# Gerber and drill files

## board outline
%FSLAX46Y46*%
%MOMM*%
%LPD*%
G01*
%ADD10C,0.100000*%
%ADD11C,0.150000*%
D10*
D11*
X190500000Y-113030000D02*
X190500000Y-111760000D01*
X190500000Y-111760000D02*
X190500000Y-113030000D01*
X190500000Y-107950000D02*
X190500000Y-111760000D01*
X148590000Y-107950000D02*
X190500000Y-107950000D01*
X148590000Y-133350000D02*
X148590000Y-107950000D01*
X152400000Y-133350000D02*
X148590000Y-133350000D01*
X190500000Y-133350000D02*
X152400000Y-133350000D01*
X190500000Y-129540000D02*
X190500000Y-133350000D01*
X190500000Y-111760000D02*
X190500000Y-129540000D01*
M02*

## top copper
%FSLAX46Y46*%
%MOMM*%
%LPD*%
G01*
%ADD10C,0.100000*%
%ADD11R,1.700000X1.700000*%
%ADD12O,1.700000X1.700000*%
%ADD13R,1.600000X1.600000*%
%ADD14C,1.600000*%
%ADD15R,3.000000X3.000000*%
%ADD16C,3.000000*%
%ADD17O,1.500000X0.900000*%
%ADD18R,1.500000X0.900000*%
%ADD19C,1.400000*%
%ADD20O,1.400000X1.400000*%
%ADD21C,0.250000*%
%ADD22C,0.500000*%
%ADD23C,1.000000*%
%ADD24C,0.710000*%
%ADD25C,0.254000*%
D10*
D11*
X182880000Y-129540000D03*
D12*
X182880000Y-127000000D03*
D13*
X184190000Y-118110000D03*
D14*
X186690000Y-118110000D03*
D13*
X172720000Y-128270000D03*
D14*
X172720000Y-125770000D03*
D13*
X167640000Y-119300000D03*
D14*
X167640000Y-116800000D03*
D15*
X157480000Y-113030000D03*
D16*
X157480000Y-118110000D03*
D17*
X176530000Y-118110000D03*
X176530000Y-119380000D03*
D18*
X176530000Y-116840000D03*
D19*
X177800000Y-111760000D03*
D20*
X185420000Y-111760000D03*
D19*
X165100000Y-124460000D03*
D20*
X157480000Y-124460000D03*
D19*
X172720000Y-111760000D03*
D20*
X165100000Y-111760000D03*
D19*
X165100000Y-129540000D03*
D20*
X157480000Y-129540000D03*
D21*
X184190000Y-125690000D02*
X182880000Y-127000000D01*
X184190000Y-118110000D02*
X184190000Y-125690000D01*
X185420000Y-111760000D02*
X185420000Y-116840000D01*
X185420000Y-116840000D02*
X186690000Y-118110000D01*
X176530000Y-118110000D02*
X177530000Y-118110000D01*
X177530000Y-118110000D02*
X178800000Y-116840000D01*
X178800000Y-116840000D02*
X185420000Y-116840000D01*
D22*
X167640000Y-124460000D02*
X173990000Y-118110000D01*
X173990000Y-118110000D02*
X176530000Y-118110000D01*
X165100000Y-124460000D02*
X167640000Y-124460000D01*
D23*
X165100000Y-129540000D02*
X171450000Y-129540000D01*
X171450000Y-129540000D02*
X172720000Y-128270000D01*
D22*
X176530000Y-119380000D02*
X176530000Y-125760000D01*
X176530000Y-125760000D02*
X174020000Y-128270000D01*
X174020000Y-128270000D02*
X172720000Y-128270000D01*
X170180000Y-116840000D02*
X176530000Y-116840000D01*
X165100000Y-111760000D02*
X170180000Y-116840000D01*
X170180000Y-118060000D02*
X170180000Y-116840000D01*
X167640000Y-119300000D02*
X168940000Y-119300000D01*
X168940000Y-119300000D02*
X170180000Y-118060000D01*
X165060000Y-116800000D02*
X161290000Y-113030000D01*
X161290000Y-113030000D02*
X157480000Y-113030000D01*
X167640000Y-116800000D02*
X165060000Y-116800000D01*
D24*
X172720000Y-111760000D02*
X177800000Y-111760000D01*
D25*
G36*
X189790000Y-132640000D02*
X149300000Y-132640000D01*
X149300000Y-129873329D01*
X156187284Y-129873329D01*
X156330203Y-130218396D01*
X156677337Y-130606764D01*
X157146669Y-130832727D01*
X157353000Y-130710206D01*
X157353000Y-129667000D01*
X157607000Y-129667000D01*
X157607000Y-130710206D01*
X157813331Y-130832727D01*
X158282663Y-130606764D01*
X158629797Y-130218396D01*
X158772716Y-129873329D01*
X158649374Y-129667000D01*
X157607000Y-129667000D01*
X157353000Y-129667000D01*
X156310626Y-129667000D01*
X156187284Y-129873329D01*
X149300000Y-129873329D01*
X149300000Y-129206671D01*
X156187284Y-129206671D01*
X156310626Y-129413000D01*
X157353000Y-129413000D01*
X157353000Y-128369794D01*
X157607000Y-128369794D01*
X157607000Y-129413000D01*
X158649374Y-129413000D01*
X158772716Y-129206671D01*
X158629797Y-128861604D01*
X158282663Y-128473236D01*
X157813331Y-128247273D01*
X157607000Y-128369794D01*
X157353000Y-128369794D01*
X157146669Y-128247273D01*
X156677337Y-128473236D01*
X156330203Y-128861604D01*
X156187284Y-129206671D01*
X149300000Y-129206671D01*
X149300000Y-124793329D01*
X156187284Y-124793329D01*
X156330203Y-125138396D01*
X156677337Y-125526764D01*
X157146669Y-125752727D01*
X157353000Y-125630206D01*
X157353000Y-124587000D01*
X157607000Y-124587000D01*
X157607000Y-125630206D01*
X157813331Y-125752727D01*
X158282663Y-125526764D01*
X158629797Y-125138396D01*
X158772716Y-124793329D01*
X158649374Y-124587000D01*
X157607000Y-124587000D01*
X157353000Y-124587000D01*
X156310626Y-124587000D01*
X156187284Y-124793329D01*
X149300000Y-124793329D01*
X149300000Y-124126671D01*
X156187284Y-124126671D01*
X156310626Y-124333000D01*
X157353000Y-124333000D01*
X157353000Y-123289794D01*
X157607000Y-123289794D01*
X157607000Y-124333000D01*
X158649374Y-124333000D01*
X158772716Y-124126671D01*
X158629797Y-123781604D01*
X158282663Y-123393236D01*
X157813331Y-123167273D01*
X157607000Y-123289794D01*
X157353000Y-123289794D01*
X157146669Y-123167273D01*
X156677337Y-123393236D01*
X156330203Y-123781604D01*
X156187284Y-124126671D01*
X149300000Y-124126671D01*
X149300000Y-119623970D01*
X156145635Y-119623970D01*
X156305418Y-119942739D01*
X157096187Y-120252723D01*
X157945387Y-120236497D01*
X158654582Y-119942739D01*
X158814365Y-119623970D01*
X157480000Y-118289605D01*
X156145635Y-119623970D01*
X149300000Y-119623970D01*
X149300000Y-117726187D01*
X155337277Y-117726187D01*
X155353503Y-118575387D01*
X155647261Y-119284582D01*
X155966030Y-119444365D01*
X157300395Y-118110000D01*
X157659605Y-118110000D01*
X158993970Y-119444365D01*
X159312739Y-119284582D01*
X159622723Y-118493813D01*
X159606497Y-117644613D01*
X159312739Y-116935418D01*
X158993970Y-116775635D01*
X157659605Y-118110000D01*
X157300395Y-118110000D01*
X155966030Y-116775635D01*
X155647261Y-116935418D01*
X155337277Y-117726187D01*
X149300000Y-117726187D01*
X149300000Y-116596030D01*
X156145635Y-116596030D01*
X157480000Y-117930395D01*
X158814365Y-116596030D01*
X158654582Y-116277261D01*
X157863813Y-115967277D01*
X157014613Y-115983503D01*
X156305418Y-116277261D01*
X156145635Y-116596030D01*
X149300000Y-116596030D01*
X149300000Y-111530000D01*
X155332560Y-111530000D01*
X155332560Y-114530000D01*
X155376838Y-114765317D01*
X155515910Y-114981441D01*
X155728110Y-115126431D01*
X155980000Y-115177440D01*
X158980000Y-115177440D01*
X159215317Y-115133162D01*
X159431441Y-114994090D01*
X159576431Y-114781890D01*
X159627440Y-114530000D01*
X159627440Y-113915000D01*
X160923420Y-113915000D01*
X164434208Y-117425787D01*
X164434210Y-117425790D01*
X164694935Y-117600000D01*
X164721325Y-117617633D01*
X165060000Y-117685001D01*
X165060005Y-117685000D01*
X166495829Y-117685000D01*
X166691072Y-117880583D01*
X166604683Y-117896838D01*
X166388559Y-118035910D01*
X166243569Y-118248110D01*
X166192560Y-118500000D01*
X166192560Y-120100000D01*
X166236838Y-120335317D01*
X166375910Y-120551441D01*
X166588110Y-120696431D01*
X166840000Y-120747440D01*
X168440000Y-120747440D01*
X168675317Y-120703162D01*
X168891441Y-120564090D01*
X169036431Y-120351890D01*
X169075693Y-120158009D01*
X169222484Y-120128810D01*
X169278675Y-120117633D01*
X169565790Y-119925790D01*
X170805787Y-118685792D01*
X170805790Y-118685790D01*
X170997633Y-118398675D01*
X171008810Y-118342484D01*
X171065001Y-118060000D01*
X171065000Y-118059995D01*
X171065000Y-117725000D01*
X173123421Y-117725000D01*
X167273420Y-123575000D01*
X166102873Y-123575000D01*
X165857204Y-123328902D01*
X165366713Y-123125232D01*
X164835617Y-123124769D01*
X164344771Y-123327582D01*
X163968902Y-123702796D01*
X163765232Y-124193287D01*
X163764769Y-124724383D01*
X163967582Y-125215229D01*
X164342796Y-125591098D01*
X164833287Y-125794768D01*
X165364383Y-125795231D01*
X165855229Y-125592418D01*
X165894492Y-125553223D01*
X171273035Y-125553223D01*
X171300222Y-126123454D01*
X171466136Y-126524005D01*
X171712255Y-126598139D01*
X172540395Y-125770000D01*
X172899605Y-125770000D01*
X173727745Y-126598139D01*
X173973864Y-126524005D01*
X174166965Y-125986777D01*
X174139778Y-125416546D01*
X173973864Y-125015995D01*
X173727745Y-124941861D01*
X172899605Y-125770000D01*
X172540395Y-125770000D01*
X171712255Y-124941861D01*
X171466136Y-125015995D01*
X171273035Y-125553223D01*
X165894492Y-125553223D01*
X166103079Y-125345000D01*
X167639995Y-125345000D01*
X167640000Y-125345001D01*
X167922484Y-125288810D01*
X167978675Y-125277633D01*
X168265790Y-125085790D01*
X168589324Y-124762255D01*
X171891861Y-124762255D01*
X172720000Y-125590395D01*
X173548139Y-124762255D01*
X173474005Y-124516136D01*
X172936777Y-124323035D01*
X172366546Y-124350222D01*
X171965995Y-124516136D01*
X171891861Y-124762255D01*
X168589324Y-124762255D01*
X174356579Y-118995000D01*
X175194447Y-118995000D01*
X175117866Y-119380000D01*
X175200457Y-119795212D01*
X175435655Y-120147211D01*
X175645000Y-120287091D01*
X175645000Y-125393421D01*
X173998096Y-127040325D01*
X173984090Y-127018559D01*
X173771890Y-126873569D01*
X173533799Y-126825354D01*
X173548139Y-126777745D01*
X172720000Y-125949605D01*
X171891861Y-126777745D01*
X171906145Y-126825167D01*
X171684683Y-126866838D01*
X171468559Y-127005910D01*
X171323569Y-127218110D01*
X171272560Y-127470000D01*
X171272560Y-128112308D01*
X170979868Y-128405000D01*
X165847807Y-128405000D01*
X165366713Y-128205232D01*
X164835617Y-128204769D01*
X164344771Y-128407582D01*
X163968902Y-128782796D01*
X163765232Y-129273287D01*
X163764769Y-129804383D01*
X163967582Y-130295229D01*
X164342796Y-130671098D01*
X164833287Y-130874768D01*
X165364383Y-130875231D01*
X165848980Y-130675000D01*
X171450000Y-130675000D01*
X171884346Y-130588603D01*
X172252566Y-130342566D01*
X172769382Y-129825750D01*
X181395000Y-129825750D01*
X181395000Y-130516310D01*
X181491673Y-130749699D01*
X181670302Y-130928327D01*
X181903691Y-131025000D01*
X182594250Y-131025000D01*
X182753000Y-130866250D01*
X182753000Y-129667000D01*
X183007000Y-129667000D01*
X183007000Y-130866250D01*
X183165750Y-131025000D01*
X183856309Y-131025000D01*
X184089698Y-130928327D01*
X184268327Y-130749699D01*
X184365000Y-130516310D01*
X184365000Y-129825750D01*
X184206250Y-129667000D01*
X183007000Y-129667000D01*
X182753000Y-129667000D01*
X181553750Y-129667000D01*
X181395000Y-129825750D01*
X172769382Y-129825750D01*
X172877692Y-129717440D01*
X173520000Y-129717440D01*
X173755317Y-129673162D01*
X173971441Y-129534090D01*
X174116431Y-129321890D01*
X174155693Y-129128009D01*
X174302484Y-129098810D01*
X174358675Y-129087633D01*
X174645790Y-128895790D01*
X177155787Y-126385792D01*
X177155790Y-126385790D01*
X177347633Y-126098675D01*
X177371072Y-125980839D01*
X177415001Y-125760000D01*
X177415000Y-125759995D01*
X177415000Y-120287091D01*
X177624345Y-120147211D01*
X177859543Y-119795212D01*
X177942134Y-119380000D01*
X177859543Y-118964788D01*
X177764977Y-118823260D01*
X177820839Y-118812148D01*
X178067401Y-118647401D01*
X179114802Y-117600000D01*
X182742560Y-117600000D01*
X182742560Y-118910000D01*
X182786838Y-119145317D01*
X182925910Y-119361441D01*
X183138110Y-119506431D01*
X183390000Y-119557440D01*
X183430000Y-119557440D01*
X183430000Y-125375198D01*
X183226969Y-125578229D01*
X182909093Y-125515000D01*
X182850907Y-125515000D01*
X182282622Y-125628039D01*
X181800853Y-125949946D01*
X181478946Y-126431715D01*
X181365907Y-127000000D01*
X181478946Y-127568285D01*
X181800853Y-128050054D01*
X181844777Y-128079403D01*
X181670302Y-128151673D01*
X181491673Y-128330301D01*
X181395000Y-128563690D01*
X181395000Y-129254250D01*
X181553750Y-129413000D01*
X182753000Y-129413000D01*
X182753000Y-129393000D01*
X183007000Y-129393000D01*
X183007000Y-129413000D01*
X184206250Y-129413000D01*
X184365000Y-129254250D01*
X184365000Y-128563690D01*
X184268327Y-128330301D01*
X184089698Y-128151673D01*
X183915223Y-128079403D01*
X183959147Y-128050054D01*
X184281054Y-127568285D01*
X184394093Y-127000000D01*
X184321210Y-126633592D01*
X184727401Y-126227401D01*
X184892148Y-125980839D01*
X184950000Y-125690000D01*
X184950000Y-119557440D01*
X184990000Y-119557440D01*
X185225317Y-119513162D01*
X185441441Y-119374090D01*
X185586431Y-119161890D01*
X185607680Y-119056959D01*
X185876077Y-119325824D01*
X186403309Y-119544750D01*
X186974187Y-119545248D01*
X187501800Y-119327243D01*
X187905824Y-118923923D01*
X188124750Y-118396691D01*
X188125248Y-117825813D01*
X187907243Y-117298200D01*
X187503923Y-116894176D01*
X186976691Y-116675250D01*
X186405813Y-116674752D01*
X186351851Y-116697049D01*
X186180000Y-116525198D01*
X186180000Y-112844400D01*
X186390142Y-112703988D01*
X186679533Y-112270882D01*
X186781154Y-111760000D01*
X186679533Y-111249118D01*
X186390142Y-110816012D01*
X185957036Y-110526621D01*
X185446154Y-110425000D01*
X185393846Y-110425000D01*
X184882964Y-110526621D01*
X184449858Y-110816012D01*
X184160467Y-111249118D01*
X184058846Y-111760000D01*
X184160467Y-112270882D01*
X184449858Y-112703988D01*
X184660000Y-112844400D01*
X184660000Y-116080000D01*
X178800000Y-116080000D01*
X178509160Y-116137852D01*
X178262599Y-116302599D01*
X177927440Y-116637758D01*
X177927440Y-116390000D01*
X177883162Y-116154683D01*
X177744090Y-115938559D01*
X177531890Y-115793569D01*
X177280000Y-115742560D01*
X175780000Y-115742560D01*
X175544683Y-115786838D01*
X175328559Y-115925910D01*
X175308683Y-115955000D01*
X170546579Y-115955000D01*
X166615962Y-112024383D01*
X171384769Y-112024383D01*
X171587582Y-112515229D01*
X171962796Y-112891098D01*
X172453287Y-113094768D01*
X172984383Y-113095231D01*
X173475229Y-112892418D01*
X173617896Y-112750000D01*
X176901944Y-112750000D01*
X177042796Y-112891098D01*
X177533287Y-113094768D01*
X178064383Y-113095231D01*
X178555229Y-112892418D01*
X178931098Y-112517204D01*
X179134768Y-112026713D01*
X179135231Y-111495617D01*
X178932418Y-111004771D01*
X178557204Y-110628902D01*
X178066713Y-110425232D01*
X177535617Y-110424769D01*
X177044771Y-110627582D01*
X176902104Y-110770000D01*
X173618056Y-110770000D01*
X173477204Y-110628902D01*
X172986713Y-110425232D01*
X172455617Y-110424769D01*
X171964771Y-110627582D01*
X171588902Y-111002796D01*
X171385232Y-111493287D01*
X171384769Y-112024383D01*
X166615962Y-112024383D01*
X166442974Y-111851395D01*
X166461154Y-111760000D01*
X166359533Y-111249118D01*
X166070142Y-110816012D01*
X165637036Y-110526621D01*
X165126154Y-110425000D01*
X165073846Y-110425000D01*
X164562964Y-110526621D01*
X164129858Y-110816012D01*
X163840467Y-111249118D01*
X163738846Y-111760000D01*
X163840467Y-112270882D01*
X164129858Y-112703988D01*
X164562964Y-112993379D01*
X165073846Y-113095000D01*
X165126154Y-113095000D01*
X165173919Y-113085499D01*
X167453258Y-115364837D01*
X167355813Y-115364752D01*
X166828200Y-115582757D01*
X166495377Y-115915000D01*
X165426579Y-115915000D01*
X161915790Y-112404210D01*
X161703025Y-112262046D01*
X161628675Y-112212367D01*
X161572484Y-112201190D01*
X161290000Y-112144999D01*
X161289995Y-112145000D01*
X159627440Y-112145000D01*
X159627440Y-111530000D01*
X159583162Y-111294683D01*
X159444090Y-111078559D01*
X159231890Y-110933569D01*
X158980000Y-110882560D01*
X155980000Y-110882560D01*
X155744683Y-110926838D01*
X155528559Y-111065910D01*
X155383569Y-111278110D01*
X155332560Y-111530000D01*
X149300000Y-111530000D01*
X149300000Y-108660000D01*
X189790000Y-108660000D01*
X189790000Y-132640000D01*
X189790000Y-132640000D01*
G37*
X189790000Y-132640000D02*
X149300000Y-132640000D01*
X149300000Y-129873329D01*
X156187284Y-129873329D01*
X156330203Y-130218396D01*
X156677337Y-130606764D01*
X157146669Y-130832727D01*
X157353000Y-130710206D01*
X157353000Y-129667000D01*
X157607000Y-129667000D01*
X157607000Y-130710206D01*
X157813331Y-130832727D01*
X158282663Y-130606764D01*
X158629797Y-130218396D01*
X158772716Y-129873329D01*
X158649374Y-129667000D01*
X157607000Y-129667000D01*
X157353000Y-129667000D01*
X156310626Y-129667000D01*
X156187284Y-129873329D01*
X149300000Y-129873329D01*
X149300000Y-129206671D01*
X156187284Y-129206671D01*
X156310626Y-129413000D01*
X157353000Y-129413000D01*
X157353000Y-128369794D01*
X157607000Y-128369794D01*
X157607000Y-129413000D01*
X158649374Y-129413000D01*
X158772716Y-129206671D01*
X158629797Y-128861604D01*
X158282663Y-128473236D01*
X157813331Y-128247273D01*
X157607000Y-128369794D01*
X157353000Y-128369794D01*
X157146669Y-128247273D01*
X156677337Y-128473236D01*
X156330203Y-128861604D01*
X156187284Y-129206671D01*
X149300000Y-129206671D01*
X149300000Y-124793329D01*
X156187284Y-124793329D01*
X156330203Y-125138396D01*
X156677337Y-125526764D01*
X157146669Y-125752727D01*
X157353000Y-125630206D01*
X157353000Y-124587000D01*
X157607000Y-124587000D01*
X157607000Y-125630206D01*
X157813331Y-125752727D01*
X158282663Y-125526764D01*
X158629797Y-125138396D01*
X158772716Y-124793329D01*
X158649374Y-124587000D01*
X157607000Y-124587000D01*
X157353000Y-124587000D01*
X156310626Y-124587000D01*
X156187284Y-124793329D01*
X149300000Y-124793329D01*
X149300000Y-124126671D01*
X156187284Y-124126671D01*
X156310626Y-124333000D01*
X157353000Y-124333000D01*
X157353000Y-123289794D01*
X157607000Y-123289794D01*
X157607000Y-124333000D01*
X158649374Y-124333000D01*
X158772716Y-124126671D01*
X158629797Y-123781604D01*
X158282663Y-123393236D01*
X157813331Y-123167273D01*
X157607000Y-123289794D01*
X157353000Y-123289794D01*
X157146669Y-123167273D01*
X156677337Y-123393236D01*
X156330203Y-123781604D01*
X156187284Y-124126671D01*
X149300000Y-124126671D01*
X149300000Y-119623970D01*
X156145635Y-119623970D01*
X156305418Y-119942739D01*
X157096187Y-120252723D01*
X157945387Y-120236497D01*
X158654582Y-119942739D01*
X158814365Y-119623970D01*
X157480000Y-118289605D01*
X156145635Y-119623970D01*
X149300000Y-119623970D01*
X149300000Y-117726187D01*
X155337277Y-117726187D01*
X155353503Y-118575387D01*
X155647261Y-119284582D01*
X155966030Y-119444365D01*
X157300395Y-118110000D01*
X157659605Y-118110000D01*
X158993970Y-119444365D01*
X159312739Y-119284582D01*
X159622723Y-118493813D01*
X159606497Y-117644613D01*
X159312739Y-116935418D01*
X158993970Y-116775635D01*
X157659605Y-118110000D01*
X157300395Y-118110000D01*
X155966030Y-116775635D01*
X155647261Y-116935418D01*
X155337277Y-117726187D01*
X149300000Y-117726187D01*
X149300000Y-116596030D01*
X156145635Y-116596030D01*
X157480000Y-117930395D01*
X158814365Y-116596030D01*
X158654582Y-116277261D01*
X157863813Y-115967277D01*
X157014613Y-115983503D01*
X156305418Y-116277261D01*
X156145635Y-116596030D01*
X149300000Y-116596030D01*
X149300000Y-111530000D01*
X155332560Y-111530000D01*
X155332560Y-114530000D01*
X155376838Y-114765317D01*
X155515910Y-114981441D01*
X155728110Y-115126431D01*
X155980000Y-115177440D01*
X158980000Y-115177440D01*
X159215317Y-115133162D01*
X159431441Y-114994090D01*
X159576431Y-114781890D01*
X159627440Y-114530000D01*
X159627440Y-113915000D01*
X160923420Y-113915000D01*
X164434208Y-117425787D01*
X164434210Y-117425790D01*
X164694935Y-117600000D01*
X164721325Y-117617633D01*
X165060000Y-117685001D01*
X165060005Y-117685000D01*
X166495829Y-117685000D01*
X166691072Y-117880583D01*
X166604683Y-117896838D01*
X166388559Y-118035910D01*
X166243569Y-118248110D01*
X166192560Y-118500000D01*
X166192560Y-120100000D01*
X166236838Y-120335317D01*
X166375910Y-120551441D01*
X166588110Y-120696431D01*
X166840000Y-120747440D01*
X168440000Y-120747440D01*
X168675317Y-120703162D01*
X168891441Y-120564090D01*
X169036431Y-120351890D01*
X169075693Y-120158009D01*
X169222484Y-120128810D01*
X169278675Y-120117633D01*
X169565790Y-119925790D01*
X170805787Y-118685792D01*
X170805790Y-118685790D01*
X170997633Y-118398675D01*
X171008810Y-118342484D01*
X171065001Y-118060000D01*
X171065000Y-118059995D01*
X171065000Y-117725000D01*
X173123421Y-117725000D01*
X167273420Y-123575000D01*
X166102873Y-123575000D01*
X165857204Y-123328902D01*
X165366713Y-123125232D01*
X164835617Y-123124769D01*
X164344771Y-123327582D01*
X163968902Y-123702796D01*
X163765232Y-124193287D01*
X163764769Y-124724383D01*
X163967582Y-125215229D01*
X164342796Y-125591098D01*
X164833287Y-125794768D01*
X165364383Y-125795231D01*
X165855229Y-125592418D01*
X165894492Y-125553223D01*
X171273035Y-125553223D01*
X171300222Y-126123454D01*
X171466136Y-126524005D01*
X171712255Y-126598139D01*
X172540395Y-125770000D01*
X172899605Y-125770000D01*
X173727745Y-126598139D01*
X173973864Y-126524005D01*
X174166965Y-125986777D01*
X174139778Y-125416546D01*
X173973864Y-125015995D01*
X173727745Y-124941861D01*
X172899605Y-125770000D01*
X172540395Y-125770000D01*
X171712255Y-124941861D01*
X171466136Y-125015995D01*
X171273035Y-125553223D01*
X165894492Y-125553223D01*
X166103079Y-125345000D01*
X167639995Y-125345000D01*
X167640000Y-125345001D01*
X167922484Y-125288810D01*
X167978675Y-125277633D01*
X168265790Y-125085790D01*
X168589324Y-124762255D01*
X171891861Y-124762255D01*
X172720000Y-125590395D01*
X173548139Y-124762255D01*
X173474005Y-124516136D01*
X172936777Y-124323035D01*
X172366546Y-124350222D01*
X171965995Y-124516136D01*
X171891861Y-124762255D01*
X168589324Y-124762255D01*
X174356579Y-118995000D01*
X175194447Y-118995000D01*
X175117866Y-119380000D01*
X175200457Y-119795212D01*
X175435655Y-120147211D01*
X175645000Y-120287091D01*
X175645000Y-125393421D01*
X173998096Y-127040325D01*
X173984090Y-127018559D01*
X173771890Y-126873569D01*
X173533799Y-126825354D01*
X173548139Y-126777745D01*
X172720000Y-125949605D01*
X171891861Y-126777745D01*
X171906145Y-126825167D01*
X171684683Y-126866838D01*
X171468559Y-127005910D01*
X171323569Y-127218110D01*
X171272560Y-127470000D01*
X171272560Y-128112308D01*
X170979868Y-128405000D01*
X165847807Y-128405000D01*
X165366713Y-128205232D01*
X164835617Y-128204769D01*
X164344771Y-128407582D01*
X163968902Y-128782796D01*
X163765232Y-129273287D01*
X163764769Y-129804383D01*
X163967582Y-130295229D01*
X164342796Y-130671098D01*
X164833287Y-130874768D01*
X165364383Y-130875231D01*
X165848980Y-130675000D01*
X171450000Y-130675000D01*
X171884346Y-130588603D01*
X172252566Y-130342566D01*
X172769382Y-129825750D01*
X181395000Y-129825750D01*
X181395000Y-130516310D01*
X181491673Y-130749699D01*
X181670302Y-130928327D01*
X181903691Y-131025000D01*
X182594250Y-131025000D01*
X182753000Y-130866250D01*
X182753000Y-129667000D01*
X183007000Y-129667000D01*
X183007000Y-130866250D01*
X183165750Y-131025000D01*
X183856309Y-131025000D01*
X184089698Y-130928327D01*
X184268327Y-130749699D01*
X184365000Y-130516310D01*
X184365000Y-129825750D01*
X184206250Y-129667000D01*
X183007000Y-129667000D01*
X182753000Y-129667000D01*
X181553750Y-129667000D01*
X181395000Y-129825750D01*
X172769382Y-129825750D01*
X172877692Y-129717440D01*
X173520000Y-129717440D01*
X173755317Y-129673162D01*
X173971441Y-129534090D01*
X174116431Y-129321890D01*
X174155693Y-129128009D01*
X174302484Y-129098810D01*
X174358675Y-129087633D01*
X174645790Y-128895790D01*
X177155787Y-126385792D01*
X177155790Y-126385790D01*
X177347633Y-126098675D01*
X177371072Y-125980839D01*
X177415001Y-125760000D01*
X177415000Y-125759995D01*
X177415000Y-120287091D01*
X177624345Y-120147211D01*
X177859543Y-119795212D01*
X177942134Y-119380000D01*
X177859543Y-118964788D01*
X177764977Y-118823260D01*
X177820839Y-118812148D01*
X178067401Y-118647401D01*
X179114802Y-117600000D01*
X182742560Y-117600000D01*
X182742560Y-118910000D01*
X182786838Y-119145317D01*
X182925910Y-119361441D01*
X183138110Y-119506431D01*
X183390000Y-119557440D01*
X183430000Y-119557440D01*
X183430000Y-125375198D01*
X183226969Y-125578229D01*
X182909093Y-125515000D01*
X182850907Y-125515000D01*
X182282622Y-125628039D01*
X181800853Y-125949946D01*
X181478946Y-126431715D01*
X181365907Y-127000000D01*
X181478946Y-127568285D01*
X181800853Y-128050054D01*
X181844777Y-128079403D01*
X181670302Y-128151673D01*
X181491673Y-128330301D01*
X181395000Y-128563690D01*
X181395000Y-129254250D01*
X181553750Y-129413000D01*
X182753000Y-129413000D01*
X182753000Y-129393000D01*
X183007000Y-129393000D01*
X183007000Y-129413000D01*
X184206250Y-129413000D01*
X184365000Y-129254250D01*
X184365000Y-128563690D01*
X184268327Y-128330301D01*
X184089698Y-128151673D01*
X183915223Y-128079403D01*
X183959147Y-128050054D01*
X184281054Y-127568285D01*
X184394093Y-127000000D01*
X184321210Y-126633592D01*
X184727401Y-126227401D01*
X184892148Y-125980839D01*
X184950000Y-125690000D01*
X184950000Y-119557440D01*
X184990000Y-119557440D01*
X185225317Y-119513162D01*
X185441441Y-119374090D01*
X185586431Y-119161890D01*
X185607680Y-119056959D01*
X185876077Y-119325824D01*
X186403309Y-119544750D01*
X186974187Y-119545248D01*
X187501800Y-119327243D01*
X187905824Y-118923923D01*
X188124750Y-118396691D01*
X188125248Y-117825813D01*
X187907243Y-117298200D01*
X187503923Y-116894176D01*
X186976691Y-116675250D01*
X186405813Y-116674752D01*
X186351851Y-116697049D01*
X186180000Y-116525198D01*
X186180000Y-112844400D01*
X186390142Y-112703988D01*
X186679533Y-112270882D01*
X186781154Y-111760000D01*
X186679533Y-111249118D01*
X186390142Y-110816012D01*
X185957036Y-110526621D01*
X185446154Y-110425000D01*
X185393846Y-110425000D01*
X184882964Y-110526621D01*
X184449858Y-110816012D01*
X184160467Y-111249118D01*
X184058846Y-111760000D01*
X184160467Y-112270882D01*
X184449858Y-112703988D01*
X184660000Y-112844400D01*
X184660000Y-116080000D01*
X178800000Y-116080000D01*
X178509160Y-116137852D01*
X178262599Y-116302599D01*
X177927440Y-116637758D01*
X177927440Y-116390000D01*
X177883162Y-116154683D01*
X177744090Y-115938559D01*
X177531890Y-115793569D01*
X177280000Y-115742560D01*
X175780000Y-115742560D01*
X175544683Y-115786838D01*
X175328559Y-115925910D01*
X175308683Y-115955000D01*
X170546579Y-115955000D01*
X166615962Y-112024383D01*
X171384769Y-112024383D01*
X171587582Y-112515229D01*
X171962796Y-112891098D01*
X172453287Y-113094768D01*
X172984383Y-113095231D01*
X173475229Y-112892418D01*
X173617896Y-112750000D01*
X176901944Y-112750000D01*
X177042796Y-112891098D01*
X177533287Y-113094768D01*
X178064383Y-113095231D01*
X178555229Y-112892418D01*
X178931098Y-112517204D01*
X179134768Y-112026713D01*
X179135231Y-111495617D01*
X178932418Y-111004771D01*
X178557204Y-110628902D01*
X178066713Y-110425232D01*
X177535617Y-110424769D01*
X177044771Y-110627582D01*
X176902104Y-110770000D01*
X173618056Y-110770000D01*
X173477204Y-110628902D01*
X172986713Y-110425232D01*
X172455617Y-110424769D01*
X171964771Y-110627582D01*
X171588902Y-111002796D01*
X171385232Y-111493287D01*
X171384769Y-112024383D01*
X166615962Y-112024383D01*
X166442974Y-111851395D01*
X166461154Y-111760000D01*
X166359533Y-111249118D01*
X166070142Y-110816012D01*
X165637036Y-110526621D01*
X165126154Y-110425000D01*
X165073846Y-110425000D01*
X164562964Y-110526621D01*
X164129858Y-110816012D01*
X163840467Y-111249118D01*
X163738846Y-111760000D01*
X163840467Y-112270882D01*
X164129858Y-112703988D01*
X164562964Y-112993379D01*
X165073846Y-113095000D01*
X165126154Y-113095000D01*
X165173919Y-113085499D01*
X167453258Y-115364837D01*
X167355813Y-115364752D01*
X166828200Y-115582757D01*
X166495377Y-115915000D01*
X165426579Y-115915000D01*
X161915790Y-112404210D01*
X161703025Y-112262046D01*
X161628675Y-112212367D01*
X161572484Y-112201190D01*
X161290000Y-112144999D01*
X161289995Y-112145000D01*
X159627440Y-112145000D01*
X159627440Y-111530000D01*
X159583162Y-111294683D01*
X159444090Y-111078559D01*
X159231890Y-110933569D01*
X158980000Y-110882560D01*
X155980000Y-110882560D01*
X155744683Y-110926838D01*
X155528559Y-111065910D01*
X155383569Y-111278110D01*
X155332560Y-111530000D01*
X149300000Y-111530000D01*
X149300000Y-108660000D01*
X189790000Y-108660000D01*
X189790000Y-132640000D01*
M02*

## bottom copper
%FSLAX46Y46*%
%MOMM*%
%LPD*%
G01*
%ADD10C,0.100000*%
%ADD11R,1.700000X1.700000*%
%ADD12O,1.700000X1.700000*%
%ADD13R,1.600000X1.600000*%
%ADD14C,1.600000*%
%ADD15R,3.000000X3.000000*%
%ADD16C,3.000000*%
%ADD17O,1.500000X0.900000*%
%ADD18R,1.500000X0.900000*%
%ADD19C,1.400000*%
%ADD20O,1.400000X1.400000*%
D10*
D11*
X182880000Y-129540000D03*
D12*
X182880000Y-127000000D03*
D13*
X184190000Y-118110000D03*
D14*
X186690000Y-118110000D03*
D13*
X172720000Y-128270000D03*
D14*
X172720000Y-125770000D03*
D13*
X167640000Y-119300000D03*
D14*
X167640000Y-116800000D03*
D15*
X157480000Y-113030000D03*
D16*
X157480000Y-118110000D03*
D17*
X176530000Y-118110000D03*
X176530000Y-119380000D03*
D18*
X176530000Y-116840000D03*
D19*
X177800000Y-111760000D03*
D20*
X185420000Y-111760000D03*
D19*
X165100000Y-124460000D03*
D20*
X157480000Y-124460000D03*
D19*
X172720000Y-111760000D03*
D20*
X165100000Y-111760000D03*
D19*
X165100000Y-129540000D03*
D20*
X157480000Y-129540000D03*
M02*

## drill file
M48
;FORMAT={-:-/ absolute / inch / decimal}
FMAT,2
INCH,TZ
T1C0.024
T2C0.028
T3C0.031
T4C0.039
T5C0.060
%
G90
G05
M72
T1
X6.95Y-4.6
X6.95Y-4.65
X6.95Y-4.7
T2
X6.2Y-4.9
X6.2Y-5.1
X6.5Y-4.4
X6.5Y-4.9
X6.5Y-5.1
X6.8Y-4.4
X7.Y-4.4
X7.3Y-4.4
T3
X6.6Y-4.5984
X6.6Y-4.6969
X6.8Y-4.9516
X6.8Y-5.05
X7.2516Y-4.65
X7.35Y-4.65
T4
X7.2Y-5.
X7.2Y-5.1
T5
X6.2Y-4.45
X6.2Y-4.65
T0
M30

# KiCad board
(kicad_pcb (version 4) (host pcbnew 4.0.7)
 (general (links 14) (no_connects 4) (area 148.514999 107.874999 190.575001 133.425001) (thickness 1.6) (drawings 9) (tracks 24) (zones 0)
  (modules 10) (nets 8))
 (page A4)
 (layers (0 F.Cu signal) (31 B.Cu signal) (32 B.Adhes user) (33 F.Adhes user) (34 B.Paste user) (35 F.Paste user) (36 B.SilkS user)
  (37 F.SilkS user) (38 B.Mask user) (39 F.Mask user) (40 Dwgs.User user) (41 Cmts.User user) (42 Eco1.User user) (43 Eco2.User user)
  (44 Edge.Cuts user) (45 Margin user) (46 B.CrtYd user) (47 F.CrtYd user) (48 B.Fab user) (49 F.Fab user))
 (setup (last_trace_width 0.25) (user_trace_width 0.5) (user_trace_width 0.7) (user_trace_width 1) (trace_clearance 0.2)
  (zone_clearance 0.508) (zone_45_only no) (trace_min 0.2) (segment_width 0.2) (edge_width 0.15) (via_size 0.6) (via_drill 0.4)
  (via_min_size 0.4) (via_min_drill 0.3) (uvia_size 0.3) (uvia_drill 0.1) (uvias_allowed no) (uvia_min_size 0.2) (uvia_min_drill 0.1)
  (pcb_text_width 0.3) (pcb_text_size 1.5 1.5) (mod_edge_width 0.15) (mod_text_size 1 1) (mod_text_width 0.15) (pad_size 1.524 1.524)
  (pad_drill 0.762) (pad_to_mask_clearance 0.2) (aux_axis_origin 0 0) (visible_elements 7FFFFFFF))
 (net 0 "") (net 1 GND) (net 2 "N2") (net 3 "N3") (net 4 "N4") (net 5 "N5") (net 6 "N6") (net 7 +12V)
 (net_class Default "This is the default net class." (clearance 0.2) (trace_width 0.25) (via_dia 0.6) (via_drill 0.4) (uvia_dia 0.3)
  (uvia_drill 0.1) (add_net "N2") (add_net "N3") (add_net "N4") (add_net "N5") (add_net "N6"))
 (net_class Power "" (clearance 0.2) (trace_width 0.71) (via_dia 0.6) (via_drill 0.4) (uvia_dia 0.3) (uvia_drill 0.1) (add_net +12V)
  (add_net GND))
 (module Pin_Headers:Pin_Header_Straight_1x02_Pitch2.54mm (layer F.Cu) (at 182.88 129.54 180)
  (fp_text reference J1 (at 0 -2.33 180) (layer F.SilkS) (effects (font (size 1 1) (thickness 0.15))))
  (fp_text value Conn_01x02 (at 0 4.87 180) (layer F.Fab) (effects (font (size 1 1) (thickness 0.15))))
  (pad 1 thru_hole rect (at 0 0 180) (size 1.7 1.7) (drill 1) (layers *.Cu *.Mask) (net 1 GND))
  (pad 2 thru_hole oval (at 0 2.54 180) (size 1.7 1.7) (drill 1) (layers *.Cu *.Mask) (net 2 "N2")))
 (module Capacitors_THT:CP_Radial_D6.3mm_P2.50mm (layer F.Cu) (at 184.19 118.11)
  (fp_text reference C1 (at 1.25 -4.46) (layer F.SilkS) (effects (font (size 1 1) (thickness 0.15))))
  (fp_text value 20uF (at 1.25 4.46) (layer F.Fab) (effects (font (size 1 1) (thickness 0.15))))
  (pad 1 thru_hole rect (at 0 0) (size 1.6 1.6) (drill 0.8) (layers *.Cu *.Mask) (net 2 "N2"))
  (pad 2 thru_hole circle (at 2.5 0) (size 1.6 1.6) (drill 0.8) (layers *.Cu *.Mask) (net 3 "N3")))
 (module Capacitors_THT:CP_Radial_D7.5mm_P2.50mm (layer F.Cu) (at 172.72 128.27 90)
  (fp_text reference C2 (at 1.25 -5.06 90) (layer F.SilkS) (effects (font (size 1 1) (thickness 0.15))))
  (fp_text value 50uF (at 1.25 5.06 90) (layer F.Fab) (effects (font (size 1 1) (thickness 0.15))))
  (pad 1 thru_hole rect (at 0 0 90) (size 1.6 1.6) (drill 0.8) (layers *.Cu *.Mask) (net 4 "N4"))
  (pad 2 thru_hole circle (at 2.5 0 90) (size 1.6 1.6) (drill 0.8) (layers *.Cu *.Mask) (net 1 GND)))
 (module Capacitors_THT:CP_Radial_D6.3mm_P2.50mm (layer F.Cu) (at 167.64 119.3 90)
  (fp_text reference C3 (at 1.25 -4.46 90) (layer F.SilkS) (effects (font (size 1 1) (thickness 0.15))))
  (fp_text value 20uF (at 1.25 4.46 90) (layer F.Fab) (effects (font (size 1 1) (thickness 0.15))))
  (pad 1 thru_hole rect (at 0 0 90) (size 1.6 1.6) (drill 0.8) (layers *.Cu *.Mask) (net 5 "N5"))
  (pad 2 thru_hole circle (at 2.5 0 90) (size 1.6 1.6) (drill 0.8) (layers *.Cu *.Mask) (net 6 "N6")))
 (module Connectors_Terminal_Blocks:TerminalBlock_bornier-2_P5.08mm (layer F.Cu) (at 157.48 113.03 270)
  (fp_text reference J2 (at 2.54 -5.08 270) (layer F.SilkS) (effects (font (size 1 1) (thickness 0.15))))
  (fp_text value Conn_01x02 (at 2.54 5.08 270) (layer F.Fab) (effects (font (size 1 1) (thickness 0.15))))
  (pad 1 thru_hole rect (at 0 0 270) (size 3 3) (drill 1.52) (layers *.Cu *.Mask) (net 6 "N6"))
  (pad 2 thru_hole circle (at 5.08 0 270) (size 3 3) (drill 1.52) (layers *.Cu *.Mask) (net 1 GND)))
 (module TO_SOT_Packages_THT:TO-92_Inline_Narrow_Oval (layer F.Cu) (at 176.53 116.84 270)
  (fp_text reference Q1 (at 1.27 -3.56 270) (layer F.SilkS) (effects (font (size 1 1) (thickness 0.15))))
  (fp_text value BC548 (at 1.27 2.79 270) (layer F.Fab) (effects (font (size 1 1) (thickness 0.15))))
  (pad 2 thru_hole oval (at 1.27 0 90) (size 0.9 1.5) (drill 0.6) (layers *.Cu *.Mask) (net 3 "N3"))
  (pad 3 thru_hole oval (at 2.54 0 90) (size 0.9 1.5) (drill 0.6) (layers *.Cu *.Mask) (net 4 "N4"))
  (pad 1 thru_hole rect (at 0 0 90) (size 0.9 1.5) (drill 0.6) (layers *.Cu *.Mask) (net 5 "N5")))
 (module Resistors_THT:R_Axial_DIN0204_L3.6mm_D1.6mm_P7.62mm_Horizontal (layer F.Cu) (at 177.8 111.76)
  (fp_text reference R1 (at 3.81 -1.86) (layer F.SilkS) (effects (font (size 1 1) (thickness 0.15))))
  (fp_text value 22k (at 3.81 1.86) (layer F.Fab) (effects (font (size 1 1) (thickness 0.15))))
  (pad 1 thru_hole circle (at 0 0) (size 1.4 1.4) (drill 0.7) (layers *.Cu *.Mask) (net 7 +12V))
  (pad 2 thru_hole oval (at 7.62 0) (size 1.4 1.4) (drill 0.7) (layers *.Cu *.Mask) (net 3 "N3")))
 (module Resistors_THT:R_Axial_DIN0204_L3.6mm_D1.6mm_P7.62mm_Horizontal (layer F.Cu) (at 165.1 124.46 180)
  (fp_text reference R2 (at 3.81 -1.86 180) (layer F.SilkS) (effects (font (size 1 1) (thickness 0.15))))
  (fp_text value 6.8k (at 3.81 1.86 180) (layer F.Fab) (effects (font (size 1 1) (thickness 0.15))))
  (pad 1 thru_hole circle (at 0 0 180) (size 1.4 1.4) (drill 0.7) (layers *.Cu *.Mask) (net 3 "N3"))
  (pad 2 thru_hole oval (at 7.62 0 180) (size 1.4 1.4) (drill 0.7) (layers *.Cu *.Mask) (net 1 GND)))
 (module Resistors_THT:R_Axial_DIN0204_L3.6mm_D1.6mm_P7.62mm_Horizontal (layer F.Cu) (at 172.72 111.76 180)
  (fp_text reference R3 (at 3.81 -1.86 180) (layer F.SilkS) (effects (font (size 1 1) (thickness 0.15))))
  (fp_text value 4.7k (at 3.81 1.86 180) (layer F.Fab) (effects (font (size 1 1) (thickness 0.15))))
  (pad 1 thru_hole circle (at 0 0 180) (size 1.4 1.4) (drill 0.7) (layers *.Cu *.Mask) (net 7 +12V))
  (pad 2 thru_hole oval (at 7.62 0 180) (size 1.4 1.4) (drill 0.7) (layers *.Cu *.Mask) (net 5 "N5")))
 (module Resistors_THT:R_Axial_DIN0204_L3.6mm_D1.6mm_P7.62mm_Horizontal (layer F.Cu) (at 165.1 129.54 180)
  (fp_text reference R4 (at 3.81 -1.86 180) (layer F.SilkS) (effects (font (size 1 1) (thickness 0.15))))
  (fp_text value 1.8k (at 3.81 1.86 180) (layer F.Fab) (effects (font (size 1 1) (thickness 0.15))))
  (pad 1 thru_hole circle (at 0 0 180) (size 1.4 1.4) (drill 0.7) (layers *.Cu *.Mask) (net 4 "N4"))
  (pad 2 thru_hole oval (at 7.62 0 180) (size 1.4 1.4) (drill 0.7) (layers *.Cu *.Mask) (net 1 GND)))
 (gr_line (start 190.5 113.03) (end 190.5 111.76) (layer Edge.Cuts) (width 0.15))
 (gr_line (start 190.5 111.76) (end 190.5 113.03) (layer Edge.Cuts) (width 0.15))
 (gr_line (start 190.5 107.95) (end 190.5 111.76) (layer Edge.Cuts) (width 0.15))
 (gr_line (start 148.59 107.95) (end 190.5 107.95) (layer Edge.Cuts) (width 0.15))
 (gr_line (start 148.59 133.35) (end 148.59 107.95) (layer Edge.Cuts) (width 0.15))
 (gr_line (start 152.4 133.35) (end 148.59 133.35) (layer Edge.Cuts) (width 0.15))
 (gr_line (start 190.5 133.35) (end 152.4 133.35) (layer Edge.Cuts) (width 0.15))
 (gr_line (start 190.5 129.54) (end 190.5 133.35) (layer Edge.Cuts) (width 0.15))
 (gr_line (start 190.5 111.76) (end 190.5 129.54) (layer Edge.Cuts) (width 0.15))
 (segment (start 184.19 125.69) (end 182.88 127) (width 0.25) (layer F.Cu) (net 2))
 (segment (start 184.19 118.11) (end 184.19 125.69) (width 0.25) (layer F.Cu) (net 2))
 (segment (start 185.42 111.76) (end 185.42 116.84) (width 0.25) (layer F.Cu) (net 3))
 (segment (start 185.42 116.84) (end 186.69 118.11) (width 0.25) (layer F.Cu) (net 3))
 (segment (start 176.53 118.11) (end 177.53 118.11) (width 0.25) (layer F.Cu) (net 3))
 (segment (start 177.53 118.11) (end 178.8 116.84) (width 0.25) (layer F.Cu) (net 3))
 (segment (start 178.8 116.84) (end 185.42 116.84) (width 0.25) (layer F.Cu) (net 3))
 (segment (start 167.64 124.46) (end 173.99 118.11) (width 0.5) (layer F.Cu) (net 3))
 (segment (start 173.99 118.11) (end 176.53 118.11) (width 0.5) (layer F.Cu) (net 3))
 (segment (start 165.1 124.46) (end 167.64 124.46) (width 0.5) (layer F.Cu) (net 3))
 (segment (start 165.1 129.54) (end 171.45 129.54) (width 1) (layer F.Cu) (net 4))
 (segment (start 171.45 129.54) (end 172.72 128.27) (width 1) (layer F.Cu) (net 4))
 (segment (start 176.53 119.38) (end 176.53 125.76) (width 0.5) (layer F.Cu) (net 4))
 (segment (start 176.53 125.76) (end 174.02 128.27) (width 0.5) (layer F.Cu) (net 4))
 (segment (start 174.02 128.27) (end 172.72 128.27) (width 0.5) (layer F.Cu) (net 4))
 (segment (start 170.18 116.84) (end 176.53 116.84) (width 0.5) (layer F.Cu) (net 5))
 (segment (start 165.1 111.76) (end 170.18 116.84) (width 0.5) (layer F.Cu) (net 5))
 (segment (start 170.18 118.06) (end 170.18 116.84) (width 0.5) (layer F.Cu) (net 5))
 (segment (start 167.64 119.3) (end 168.94 119.3) (width 0.5) (layer F.Cu) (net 5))
 (segment (start 168.94 119.3) (end 170.18 118.06) (width 0.5) (layer F.Cu) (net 5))
 (segment (start 165.06 116.8) (end 161.29 113.03) (width 0.5) (layer F.Cu) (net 6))
 (segment (start 161.29 113.03) (end 157.48 113.03) (width 0.5) (layer F.Cu) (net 6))
 (segment (start 167.64 116.8) (end 165.06 116.8) (width 0.5) (layer F.Cu) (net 6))
 (segment (start 172.72 111.76) (end 177.8 111.76) (width 0.71) (layer F.Cu) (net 7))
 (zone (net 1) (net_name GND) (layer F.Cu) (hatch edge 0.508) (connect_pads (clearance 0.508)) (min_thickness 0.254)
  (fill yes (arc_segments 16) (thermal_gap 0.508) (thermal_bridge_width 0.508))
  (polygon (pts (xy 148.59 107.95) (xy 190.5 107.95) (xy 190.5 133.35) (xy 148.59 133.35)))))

